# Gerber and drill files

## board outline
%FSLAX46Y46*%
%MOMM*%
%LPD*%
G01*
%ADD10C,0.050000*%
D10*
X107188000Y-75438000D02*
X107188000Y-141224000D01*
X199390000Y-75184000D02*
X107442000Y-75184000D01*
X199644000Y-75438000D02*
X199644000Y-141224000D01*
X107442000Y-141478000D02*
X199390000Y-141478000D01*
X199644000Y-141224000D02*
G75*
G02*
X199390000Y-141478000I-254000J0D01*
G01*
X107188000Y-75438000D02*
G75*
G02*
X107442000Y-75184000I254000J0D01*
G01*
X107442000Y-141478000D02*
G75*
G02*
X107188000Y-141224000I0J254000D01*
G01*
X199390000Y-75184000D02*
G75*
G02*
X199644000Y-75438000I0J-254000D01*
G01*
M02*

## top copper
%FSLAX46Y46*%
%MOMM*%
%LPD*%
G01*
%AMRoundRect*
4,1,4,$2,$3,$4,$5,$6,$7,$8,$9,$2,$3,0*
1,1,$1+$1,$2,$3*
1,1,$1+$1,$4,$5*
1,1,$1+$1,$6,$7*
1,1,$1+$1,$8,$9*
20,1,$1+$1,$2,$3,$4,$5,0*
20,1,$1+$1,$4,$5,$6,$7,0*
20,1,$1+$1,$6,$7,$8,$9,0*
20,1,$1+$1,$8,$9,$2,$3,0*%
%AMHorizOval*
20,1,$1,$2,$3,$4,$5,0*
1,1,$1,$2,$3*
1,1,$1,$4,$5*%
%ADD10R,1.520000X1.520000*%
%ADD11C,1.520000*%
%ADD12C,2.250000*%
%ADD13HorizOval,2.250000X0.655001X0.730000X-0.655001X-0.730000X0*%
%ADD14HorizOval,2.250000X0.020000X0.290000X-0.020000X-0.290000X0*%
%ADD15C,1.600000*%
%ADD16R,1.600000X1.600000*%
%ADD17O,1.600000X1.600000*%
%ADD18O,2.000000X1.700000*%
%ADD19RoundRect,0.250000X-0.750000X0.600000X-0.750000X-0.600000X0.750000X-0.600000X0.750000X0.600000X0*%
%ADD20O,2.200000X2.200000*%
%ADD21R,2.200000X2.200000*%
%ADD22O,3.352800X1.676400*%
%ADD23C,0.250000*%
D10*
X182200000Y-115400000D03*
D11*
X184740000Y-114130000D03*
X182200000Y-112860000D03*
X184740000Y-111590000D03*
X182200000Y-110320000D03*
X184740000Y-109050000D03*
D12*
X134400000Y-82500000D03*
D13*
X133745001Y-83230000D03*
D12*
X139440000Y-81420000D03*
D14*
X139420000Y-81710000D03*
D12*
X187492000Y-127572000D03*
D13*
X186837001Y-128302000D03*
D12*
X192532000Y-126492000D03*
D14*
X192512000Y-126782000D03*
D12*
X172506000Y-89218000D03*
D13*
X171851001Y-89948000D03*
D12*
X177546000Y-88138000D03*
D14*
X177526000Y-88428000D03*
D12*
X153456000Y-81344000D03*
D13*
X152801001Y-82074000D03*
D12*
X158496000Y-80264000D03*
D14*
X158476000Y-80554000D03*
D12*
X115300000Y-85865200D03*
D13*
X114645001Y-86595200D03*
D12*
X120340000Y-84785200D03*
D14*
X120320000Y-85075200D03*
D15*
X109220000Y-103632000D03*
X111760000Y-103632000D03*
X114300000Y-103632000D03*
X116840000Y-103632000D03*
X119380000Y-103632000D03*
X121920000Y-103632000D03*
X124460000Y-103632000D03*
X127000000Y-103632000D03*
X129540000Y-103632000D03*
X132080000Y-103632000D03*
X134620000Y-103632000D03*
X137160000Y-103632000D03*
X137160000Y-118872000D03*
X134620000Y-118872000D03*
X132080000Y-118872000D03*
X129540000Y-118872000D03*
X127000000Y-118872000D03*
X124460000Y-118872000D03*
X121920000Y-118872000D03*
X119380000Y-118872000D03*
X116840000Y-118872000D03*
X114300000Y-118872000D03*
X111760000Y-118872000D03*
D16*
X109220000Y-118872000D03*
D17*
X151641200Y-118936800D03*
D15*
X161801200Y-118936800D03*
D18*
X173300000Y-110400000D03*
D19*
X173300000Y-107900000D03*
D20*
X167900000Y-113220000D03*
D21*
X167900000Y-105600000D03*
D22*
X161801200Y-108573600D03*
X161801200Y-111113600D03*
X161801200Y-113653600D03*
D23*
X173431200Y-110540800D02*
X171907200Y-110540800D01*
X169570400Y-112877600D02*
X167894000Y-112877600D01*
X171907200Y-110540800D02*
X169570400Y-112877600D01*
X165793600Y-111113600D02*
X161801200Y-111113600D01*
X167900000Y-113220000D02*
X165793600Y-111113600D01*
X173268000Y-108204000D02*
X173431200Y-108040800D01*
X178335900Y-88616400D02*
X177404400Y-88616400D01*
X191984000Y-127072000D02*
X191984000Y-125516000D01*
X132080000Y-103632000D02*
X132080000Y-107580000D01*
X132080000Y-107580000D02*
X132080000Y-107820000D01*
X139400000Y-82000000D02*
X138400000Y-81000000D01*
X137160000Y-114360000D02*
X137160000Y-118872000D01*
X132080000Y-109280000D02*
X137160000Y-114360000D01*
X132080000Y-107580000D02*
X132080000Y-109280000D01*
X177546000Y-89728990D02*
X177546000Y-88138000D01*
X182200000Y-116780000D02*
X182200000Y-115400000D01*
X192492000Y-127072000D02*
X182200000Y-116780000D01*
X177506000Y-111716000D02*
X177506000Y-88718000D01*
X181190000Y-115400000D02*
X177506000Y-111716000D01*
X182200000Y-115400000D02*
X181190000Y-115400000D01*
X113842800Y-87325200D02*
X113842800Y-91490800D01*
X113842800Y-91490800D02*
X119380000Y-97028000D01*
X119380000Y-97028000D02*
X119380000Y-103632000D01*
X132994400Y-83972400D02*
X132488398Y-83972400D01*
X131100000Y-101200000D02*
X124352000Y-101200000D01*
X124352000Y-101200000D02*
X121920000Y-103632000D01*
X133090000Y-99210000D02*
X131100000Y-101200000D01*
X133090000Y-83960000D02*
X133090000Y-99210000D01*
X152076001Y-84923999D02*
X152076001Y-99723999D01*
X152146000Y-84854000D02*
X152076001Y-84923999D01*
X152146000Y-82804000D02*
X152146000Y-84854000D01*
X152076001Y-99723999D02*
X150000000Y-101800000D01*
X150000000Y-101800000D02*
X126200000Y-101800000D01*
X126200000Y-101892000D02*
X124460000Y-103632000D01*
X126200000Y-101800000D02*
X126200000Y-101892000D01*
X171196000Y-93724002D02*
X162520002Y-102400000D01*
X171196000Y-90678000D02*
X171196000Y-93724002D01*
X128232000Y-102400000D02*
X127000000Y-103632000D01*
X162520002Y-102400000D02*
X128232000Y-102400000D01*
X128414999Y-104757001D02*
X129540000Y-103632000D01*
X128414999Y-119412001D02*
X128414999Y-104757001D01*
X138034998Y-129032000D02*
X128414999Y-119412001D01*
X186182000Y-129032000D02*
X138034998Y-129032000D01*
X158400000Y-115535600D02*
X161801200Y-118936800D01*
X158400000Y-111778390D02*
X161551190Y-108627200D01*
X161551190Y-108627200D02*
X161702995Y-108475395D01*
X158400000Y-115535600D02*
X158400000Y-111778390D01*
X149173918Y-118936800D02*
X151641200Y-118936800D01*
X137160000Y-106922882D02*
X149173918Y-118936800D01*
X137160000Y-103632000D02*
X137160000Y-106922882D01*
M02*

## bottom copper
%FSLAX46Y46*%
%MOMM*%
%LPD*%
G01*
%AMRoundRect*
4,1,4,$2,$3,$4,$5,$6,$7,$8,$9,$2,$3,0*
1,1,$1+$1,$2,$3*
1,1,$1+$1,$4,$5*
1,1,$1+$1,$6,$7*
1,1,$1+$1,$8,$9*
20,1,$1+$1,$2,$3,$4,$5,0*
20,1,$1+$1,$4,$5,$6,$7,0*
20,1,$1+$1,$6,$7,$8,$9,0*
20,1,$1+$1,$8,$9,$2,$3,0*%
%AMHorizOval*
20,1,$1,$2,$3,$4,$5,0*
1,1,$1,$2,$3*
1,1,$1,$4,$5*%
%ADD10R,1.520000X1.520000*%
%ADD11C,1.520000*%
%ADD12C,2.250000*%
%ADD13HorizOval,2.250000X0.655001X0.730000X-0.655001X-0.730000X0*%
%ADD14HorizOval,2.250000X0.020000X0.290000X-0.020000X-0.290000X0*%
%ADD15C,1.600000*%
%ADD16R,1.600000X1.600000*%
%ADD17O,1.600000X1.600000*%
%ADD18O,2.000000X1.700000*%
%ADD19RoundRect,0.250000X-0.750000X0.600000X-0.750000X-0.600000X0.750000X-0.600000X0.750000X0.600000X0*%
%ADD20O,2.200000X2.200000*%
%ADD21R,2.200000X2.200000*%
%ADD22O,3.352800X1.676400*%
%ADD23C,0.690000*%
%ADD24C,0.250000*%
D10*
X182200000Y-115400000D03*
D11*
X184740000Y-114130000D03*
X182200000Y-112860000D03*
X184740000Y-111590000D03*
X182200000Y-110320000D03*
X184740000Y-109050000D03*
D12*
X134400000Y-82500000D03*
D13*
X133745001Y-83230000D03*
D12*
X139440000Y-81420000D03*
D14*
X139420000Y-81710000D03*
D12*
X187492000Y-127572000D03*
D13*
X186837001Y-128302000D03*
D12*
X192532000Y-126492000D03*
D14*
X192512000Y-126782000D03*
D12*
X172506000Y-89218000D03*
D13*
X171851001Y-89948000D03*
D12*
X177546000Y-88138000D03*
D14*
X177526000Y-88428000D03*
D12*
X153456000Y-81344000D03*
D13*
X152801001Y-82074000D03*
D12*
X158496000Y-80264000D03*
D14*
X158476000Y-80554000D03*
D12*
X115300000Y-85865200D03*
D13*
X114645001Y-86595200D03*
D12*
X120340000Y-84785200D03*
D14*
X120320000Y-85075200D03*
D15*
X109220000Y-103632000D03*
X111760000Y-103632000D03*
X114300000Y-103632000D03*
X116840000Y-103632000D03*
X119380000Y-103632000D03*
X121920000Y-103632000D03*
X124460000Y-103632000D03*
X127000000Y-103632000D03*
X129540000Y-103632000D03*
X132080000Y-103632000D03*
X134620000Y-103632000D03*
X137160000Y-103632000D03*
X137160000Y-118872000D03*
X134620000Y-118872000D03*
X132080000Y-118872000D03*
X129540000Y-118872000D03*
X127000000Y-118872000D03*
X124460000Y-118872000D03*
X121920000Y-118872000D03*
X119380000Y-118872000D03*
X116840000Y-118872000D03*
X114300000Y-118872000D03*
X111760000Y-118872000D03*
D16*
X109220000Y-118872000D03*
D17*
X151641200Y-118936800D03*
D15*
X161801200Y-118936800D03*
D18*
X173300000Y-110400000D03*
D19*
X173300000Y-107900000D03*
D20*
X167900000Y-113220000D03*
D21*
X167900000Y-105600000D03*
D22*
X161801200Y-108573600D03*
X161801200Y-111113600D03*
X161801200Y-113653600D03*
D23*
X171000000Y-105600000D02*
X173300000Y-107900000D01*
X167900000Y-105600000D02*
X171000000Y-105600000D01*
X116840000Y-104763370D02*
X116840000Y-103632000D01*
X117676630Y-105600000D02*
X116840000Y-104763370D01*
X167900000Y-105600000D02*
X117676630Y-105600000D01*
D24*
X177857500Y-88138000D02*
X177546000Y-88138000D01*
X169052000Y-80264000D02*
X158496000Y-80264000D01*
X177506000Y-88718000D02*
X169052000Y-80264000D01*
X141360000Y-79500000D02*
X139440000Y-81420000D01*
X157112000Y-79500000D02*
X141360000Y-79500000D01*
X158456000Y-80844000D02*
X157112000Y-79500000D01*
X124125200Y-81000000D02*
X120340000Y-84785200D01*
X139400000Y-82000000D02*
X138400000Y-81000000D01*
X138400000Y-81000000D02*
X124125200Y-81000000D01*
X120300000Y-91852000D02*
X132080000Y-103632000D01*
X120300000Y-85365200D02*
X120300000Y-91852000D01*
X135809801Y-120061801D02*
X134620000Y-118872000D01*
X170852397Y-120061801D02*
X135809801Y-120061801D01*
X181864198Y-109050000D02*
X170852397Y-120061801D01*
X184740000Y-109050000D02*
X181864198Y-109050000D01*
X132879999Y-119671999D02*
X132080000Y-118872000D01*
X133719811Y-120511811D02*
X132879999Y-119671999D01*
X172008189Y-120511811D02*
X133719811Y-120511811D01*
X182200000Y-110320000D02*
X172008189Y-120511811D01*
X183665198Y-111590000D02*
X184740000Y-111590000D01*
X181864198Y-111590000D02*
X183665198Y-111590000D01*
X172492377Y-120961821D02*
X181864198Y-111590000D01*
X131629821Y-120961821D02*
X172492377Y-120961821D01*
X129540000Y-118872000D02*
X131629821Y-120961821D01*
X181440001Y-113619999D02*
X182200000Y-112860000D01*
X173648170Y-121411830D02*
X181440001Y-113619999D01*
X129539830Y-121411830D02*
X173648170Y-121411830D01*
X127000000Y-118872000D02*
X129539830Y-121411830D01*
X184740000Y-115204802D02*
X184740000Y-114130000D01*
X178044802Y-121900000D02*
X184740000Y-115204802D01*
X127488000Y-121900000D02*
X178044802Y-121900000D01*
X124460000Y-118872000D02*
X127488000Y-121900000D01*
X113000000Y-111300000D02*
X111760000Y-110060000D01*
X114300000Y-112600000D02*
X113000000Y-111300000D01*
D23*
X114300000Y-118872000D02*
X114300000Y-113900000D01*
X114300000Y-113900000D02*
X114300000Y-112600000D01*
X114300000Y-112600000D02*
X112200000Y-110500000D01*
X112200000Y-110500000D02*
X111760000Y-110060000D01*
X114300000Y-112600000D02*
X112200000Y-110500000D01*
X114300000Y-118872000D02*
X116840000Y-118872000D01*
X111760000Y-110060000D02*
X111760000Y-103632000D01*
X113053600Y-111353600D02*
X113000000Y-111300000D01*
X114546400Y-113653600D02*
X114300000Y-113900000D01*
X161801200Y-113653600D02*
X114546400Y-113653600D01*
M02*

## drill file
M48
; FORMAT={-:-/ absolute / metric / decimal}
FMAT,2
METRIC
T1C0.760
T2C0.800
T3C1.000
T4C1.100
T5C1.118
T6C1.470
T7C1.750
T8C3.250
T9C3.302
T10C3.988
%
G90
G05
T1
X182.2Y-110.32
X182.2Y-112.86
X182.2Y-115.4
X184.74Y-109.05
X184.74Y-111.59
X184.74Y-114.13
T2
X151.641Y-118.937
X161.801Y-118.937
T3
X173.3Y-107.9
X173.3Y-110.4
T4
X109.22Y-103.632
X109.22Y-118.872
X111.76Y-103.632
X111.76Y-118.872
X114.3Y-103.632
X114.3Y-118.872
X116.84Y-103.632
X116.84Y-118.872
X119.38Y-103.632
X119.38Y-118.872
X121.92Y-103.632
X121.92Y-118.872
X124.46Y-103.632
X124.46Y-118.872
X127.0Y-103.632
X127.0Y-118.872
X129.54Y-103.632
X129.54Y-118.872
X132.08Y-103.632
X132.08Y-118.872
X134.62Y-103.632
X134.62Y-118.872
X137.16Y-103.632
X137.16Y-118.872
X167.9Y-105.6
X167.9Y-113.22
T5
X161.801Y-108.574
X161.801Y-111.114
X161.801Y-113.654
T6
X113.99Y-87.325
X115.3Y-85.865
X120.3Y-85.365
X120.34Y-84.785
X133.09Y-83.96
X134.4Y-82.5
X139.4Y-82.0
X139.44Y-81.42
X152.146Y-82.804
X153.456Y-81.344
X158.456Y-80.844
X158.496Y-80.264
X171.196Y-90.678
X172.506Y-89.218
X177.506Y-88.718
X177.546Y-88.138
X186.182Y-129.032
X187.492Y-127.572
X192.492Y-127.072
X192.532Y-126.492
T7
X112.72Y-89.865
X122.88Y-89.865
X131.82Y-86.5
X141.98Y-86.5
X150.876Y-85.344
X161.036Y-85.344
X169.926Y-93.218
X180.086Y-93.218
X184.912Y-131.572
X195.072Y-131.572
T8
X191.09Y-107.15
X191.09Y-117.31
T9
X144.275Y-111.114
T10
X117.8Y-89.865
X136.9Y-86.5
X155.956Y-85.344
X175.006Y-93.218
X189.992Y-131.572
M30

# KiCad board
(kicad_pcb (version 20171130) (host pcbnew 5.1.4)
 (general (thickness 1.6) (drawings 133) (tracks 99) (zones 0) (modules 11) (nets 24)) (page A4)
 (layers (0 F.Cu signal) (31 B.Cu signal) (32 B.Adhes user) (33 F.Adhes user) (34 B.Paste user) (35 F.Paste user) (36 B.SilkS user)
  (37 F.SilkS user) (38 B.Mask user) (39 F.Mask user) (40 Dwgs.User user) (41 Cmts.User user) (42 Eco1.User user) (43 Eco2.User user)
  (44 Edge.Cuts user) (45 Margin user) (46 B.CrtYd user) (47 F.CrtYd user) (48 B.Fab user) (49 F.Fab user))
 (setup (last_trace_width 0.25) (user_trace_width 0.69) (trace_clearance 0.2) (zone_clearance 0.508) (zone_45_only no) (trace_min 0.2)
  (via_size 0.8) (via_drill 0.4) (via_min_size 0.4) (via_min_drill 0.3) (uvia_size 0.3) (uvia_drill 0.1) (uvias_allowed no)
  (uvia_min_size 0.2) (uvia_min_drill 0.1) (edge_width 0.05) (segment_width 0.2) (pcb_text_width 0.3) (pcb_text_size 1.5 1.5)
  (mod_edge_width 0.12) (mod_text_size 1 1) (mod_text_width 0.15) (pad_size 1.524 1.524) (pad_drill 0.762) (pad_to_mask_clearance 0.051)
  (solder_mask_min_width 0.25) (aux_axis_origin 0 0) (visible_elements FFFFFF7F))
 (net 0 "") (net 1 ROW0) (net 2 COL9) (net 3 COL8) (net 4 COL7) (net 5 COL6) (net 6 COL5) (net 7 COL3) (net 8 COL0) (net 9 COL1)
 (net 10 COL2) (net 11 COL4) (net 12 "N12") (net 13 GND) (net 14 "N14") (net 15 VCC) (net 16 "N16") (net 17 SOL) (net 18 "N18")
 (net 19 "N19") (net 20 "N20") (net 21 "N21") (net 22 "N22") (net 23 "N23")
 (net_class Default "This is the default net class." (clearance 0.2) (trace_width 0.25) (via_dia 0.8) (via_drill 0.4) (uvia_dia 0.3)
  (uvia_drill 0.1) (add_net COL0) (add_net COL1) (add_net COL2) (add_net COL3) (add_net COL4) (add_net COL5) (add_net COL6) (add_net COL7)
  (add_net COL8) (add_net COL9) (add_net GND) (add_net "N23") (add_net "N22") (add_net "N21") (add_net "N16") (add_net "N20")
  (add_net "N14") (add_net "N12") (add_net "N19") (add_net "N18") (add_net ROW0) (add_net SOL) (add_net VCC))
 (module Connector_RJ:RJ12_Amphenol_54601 (layer F.Cu) (at 182.2 115.4 90)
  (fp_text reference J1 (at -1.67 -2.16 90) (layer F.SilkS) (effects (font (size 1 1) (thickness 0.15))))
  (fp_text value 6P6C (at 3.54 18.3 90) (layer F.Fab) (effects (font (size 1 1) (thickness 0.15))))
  (pad 1 thru_hole rect (at 0 0 90) (size 1.52 1.52) (drill 0.76) (layers *.Cu *.Mask) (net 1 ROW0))
  (pad "" np_thru_hole circle (at -1.91 8.89 90) (size 3.25 3.25) (drill 3.25) (layers *.Cu *.Mask))
  (pad 2 thru_hole circle (at 1.27 2.54 90) (size 1.52 1.52) (drill 0.76) (layers *.Cu *.Mask) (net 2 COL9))
  (pad 3 thru_hole circle (at 2.54 0 90) (size 1.52 1.52) (drill 0.76) (layers *.Cu *.Mask) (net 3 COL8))
  (pad 4 thru_hole circle (at 3.81 2.54 90) (size 1.52 1.52) (drill 0.76) (layers *.Cu *.Mask) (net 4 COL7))
  (pad 5 thru_hole circle (at 5.08 0 90) (size 1.52 1.52) (drill 0.76) (layers *.Cu *.Mask) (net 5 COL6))
  (pad 6 thru_hole circle (at 6.35 2.54 90) (size 1.52 1.52) (drill 0.76) (layers *.Cu *.Mask) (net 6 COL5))
  (pad "" np_thru_hole circle (at 8.25 8.89 90) (size 3.25 3.25) (drill 3.25) (layers *.Cu *.Mask)))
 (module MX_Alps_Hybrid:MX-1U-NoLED (layer F.Cu) (at 136.9 86.5)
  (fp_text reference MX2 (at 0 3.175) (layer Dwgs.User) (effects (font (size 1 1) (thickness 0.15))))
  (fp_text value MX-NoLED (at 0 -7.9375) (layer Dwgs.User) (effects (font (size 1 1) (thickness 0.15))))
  (pad "" np_thru_hole circle (at 5.08 0 48.0996) (size 1.75 1.75) (drill 1.75) (layers *.Cu *.Mask))
  (pad "" np_thru_hole circle (at -5.08 0 48.0996) (size 1.75 1.75) (drill 1.75) (layers *.Cu *.Mask))
  (pad 1 thru_hole circle (at -2.5 -4) (size 2.25 2.25) (drill 1.47) (layers *.Cu B.Mask) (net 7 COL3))
  (pad "" np_thru_hole circle (at 0 0) (size 3.9878 3.9878) (drill 3.9878) (layers *.Cu *.Mask))
  (pad 1 thru_hole oval (at -3.81 -2.54 48.0996) (size 4.211556 2.25) (drill 1.47 (offset 0.980778 0)) (layers *.Cu B.Mask) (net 7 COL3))
  (pad 2 thru_hole circle (at 2.54 -5.08) (size 2.25 2.25) (drill 1.47) (layers *.Cu B.Mask) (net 1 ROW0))
  (pad 2 thru_hole oval (at 2.5 -4.5 86.0548) (size 2.831378 2.25) (drill 1.47 (offset 0.290689 0)) (layers *.Cu B.Mask) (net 1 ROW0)))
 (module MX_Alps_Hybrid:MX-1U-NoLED (layer F.Cu) (at 189.992 131.572)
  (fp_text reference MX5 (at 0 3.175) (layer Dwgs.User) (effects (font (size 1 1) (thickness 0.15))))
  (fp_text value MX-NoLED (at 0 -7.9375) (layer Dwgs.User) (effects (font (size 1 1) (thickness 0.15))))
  (pad "" np_thru_hole circle (at 5.08 0 48.0996) (size 1.75 1.75) (drill 1.75) (layers *.Cu *.Mask))
  (pad "" np_thru_hole circle (at -5.08 0 48.0996) (size 1.75 1.75) (drill 1.75) (layers *.Cu *.Mask))
  (pad 1 thru_hole circle (at -2.5 -4) (size 2.25 2.25) (drill 1.47) (layers *.Cu B.Mask) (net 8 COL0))
  (pad "" np_thru_hole circle (at 0 0) (size 3.9878 3.9878) (drill 3.9878) (layers *.Cu *.Mask))
  (pad 1 thru_hole oval (at -3.81 -2.54 48.0996) (size 4.211556 2.25) (drill 1.47 (offset 0.980778 0)) (layers *.Cu B.Mask) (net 8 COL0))
  (pad 2 thru_hole circle (at 2.54 -5.08) (size 2.25 2.25) (drill 1.47) (layers *.Cu B.Mask) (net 1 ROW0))
  (pad 2 thru_hole oval (at 2.5 -4.5 86.0548) (size 2.831378 2.25) (drill 1.47 (offset 0.290689 0)) (layers *.Cu B.Mask) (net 1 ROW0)))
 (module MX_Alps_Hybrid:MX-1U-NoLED (layer F.Cu) (at 175.006 93.218)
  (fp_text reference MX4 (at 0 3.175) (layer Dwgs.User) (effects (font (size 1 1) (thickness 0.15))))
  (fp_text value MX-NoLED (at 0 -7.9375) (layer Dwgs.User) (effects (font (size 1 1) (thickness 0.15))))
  (pad "" np_thru_hole circle (at 5.08 0 48.0996) (size 1.75 1.75) (drill 1.75) (layers *.Cu *.Mask))
  (pad "" np_thru_hole circle (at -5.08 0 48.0996) (size 1.75 1.75) (drill 1.75) (layers *.Cu *.Mask))
  (pad 1 thru_hole circle (at -2.5 -4) (size 2.25 2.25) (drill 1.47) (layers *.Cu B.Mask) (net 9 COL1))
  (pad "" np_thru_hole circle (at 0 0) (size 3.9878 3.9878) (drill 3.9878) (layers *.Cu *.Mask))
  (pad 1 thru_hole oval (at -3.81 -2.54 48.0996) (size 4.211556 2.25) (drill 1.47 (offset 0.980778 0)) (layers *.Cu B.Mask) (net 9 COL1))
  (pad 2 thru_hole circle (at 2.54 -5.08) (size 2.25 2.25) (drill 1.47) (layers *.Cu B.Mask) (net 1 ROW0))
  (pad 2 thru_hole oval (at 2.5 -4.5 86.0548) (size 2.831378 2.25) (drill 1.47 (offset 0.290689 0)) (layers *.Cu B.Mask) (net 1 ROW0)))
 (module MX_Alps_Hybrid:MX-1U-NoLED (layer F.Cu) (at 155.956 85.344)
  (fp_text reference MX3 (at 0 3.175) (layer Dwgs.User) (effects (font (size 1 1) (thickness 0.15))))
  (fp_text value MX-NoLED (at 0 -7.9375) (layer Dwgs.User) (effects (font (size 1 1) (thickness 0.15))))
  (pad "" np_thru_hole circle (at 5.08 0 48.0996) (size 1.75 1.75) (drill 1.75) (layers *.Cu *.Mask))
  (pad "" np_thru_hole circle (at -5.08 0 48.0996) (size 1.75 1.75) (drill 1.75) (layers *.Cu *.Mask))
  (pad 1 thru_hole circle (at -2.5 -4) (size 2.25 2.25) (drill 1.47) (layers *.Cu B.Mask) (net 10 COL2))
  (pad "" np_thru_hole circle (at 0 0) (size 3.9878 3.9878) (drill 3.9878) (layers *.Cu *.Mask))
  (pad 1 thru_hole oval (at -3.81 -2.54 48.0996) (size 4.211556 2.25) (drill 1.47 (offset 0.980778 0)) (layers *.Cu B.Mask) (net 10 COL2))
  (pad 2 thru_hole circle (at 2.54 -5.08) (size 2.25 2.25) (drill 1.47) (layers *.Cu B.Mask) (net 1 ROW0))
  (pad 2 thru_hole oval (at 2.5 -4.5 86.0548) (size 2.831378 2.25) (drill 1.47 (offset 0.290689 0)) (layers *.Cu B.Mask) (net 1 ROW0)))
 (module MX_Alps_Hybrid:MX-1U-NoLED (layer F.Cu) (at 117.8 89.8652)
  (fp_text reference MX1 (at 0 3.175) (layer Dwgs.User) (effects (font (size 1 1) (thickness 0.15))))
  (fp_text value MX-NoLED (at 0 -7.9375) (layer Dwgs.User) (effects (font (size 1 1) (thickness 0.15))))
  (pad "" np_thru_hole circle (at 5.08 0 48.0996) (size 1.75 1.75) (drill 1.75) (layers *.Cu *.Mask))
  (pad "" np_thru_hole circle (at -5.08 0 48.0996) (size 1.75 1.75) (drill 1.75) (layers *.Cu *.Mask))
  (pad 1 thru_hole circle (at -2.5 -4) (size 2.25 2.25) (drill 1.47) (layers *.Cu B.Mask) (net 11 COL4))
  (pad "" np_thru_hole circle (at 0 0) (size 3.9878 3.9878) (drill 3.9878) (layers *.Cu *.Mask))
  (pad 1 thru_hole oval (at -3.81 -2.54 48.0996) (size 4.211556 2.25) (drill 1.47 (offset 0.980778 0)) (layers *.Cu B.Mask) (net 11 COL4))
  (pad 2 thru_hole circle (at 2.54 -5.08) (size 2.25 2.25) (drill 1.47) (layers *.Cu B.Mask) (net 1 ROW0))
  (pad 2 thru_hole oval (at 2.5 -4.5 86.0548) (size 2.831378 2.25) (drill 1.47 (offset 0.290689 0)) (layers *.Cu B.Mask) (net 1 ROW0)))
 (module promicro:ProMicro (layer F.Cu) (at 123.19 111.252)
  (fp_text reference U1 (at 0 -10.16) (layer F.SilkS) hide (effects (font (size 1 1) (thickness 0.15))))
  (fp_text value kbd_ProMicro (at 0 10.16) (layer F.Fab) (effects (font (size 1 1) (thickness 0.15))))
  (pad 24 thru_hole circle (at -13.97 -7.62) (size 1.6 1.6) (drill 1.1) (layers *.Cu *.Mask F.SilkS) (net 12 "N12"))
  (pad 23 thru_hole circle (at -11.43 -7.62) (size 1.6 1.6) (drill 1.1) (layers *.Cu *.Mask F.SilkS) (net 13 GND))
  (pad 22 thru_hole circle (at -8.89 -7.62) (size 1.6 1.6) (drill 1.1) (layers *.Cu *.Mask F.SilkS) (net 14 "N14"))
  (pad 21 thru_hole circle (at -6.35 -7.62) (size 1.6 1.6) (drill 1.1) (layers *.Cu *.Mask F.SilkS) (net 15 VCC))
  (pad 20 thru_hole circle (at -3.81 -7.62) (size 1.6 1.6) (drill 1.1) (layers *.Cu *.Mask F.SilkS) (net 11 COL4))
  (pad 19 thru_hole circle (at -1.27 -7.62) (size 1.6 1.6) (drill 1.1) (layers *.Cu *.Mask F.SilkS) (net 7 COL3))
  (pad 18 thru_hole circle (at 1.27 -7.62) (size 1.6 1.6) (drill 1.1) (layers *.Cu *.Mask F.SilkS) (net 10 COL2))
  (pad 17 thru_hole circle (at 3.81 -7.62) (size 1.6 1.6) (drill 1.1) (layers *.Cu *.Mask F.SilkS) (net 9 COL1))
  (pad 16 thru_hole circle (at 6.35 -7.62) (size 1.6 1.6) (drill 1.1) (layers *.Cu *.Mask F.SilkS) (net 8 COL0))
  (pad 15 thru_hole circle (at 8.89 -7.62) (size 1.6 1.6) (drill 1.1) (layers *.Cu *.Mask F.SilkS) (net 1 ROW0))
  (pad 14 thru_hole circle (at 11.43 -7.62) (size 1.6 1.6) (drill 1.1) (layers *.Cu *.Mask F.SilkS) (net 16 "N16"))
  (pad 13 thru_hole circle (at 13.97 -7.62) (size 1.6 1.6) (drill 1.1) (layers *.Cu *.Mask F.SilkS) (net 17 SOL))
  (pad 12 thru_hole circle (at 13.97 7.62) (size 1.6 1.6) (drill 1.1) (layers *.Cu *.Mask F.SilkS) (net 1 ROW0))
  (pad 11 thru_hole circle (at 11.43 7.62) (size 1.6 1.6) (drill 1.1) (layers *.Cu *.Mask F.SilkS) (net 6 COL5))
  (pad 10 thru_hole circle (at 8.89 7.62) (size 1.6 1.6) (drill 1.1) (layers *.Cu *.Mask F.SilkS) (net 5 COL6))
  (pad 9 thru_hole circle (at 6.35 7.62) (size 1.6 1.6) (drill 1.1) (layers *.Cu *.Mask F.SilkS) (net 4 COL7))
  (pad 8 thru_hole circle (at 3.81 7.62) (size 1.6 1.6) (drill 1.1) (layers *.Cu *.Mask F.SilkS) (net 3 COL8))
  (pad 7 thru_hole circle (at 1.27 7.62) (size 1.6 1.6) (drill 1.1) (layers *.Cu *.Mask F.SilkS) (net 2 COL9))
  (pad 6 thru_hole circle (at -1.27 7.62) (size 1.6 1.6) (drill 1.1) (layers *.Cu *.Mask F.SilkS) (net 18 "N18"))
  (pad 5 thru_hole circle (at -3.81 7.62) (size 1.6 1.6) (drill 1.1) (layers *.Cu *.Mask F.SilkS) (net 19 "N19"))
  (pad 4 thru_hole circle (at -6.35 7.62) (size 1.6 1.6) (drill 1.1) (layers *.Cu *.Mask F.SilkS) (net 13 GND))
  (pad 3 thru_hole circle (at -8.89 7.62) (size 1.6 1.6) (drill 1.1) (layers *.Cu *.Mask F.SilkS) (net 13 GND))
  (pad 2 thru_hole circle (at -11.43 7.62) (size 1.6 1.6) (drill 1.1) (layers *.Cu *.Mask F.SilkS) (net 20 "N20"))
  (pad 1 thru_hole rect (at -13.97 7.62) (size 1.6 1.6) (drill 1.1) (layers *.Cu *.Mask F.SilkS) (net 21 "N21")))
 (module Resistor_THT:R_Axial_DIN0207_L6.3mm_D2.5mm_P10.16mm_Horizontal (layer B.Cu) (at 161.8012 118.9368 180)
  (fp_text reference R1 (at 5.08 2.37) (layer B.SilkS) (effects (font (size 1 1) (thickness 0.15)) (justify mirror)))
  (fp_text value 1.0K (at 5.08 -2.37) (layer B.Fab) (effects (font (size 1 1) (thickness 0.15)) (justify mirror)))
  (pad 2 thru_hole oval (at 10.16 0 180) (size 1.6 1.6) (drill 0.8) (layers *.Cu *.Mask) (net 17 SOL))
  (pad 1 thru_hole circle (at 0 0 180) (size 1.6 1.6) (drill 0.8) (layers *.Cu *.Mask) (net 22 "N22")))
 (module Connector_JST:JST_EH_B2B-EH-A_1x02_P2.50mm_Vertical (layer B.Cu) (at 173.3 107.9 270)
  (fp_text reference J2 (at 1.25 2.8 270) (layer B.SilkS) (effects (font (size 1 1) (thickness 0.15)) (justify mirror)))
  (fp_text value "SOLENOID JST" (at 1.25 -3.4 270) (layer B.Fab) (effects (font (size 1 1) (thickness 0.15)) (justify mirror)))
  (pad 2 thru_hole oval (at 2.5 0 270) (size 1.7 2) (drill 1) (layers *.Cu *.Mask) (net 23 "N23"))
  (pad 1 thru_hole roundrect (at 0 0 270) (size 1.7 2) (drill 1) (layers *.Cu *.Mask) (roundrect_rratio 0.147059) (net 15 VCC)))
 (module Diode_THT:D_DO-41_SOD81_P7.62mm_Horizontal (layer B.Cu) (at 167.9 105.6 270)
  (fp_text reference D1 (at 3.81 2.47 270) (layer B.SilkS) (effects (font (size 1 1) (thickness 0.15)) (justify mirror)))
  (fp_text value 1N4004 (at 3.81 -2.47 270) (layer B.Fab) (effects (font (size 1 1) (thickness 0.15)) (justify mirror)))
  (pad 2 thru_hole oval (at 7.62 0 270) (size 2.2 2.2) (drill 1.1) (layers *.Cu *.Mask) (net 23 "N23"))
  (pad 1 thru_hole rect (at 0 0 270) (size 2.2 2.2) (drill 1.1) (layers *.Cu *.Mask) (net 15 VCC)))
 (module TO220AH (layer B.Cu) (at 155.4512 111.1136 270)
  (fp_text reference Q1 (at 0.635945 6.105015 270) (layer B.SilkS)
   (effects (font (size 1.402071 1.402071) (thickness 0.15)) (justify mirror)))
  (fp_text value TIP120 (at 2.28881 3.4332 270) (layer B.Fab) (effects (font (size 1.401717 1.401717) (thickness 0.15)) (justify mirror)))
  (pad B thru_hole oval (at -2.54 -6.35 270) (size 1.6764 3.3528) (drill 1.1176) (layers *.Cu *.Mask) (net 22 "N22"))
  (pad C thru_hole oval (at 0 -6.35 270) (size 1.6764 3.3528) (drill 1.1176) (layers *.Cu *.Mask) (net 23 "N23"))
  (pad E thru_hole oval (at 2.54 -6.35 270) (size 1.6764 3.3528) (drill 1.1176) (layers *.Cu *.Mask) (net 13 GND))
  (pad None np_thru_hole circle (at 0 11.176 270) (size 3.302 3.302) (drill 3.302) (layers *.Cu *.Mask)))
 (gr_line (start 107.188 75.438) (end 107.188 141.224) (layer Edge.Cuts) (width 0.05))
 (gr_line (start 199.39 75.184) (end 107.442 75.184) (layer Edge.Cuts) (width 0.05))
 (gr_line (start 199.644 75.438) (end 199.644 141.224) (layer Edge.Cuts) (width 0.05))
 (gr_line (start 107.442 141.478) (end 199.39 141.478) (layer Edge.Cuts) (width 0.05))
 (gr_arc (start 199.39 141.224) (end 199.39 141.478) (angle -90) (layer Edge.Cuts) (width 0.05))
 (gr_arc (start 107.442 75.438) (end 107.442 75.184) (angle -90) (layer Edge.Cuts) (width 0.05))
 (gr_arc (start 107.442 141.224) (end 107.188 141.224) (angle -90) (layer Edge.Cuts) (width 0.05))
 (gr_arc (start 199.39 75.438) (end 199.644 75.438) (angle -90) (layer Edge.Cuts) (width 0.05))
 (segment (start 173.4312 110.5408) (end 171.9072 110.5408) (width 0.25) (layer F.Cu) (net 23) (status 10))
 (segment (start 169.5704 112.8776) (end 167.894 112.8776) (width 0.25) (layer F.Cu) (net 23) (status 20))
 (segment (start 171.9072 110.5408) (end 169.5704 112.8776) (width 0.25) (layer F.Cu) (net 23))
 (segment (start 165.7936 111.1136) (end 161.8012 111.1136) (width 0.25) (layer F.Cu) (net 23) (status 20))
 (segment (start 167.9 113.22) (end 165.7936 111.1136) (width 0.25) (layer F.Cu) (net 23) (status 10))
 (segment (start 173.268 108.204) (end 173.4312 108.0408) (width 0.25) (layer F.Cu) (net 15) (status 30))
 (segment (start 171 105.6) (end 173.3 107.9) (width 0.69) (layer B.Cu) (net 15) (status 20))
 (segment (start 167.9 105.6) (end 171 105.6) (width 0.69) (layer B.Cu) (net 15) (status 10))
 (segment (start 116.84 104.76337) (end 116.84 103.632) (width 0.69) (layer B.Cu) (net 15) (status 20))
 (segment (start 117.67663 105.6) (end 116.84 104.76337) (width 0.69) (layer B.Cu) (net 15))
 (segment (start 167.9 105.6) (end 117.67663 105.6) (width 0.69) (layer B.Cu) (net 15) (status 10))
 (segment (start 178.3359 88.6164) (end 177.4044 88.6164) (width 0.25) (layer F.Cu) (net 1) (status 30))
 (segment (start 191.984 127.072) (end 191.984 125.516) (width 0.25) (layer F.Cu) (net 1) (status 30))
 (segment (start 132.08 103.632) (end 132.08 107.58) (width 0.25) (layer F.Cu) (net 1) (status 10))
 (segment (start 132.08 107.58) (end 132.08 107.82) (width 0.25) (layer F.Cu) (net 1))
 (segment (start 139.4 82) (end 138.4 81) (width 0.25) (layer F.Cu) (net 1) (status 30))
 (segment (start 177.8575 88.138) (end 177.546 88.138) (width 0.25) (layer B.Cu) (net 1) (status 30))
 (segment (start 169.052 80.264) (end 158.496 80.264) (width 0.25) (layer B.Cu) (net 1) (status 20))
 (segment (start 177.506 88.718) (end 169.052 80.264) (width 0.25) (layer B.Cu) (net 1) (status 10))
 (segment (start 141.36 79.5) (end 139.44 81.42) (width 0.25) (layer B.Cu) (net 1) (status 20))
 (segment (start 157.112 79.5) (end 141.36 79.5) (width 0.25) (layer B.Cu) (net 1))
 (segment (start 158.456 80.844) (end 157.112 79.5) (width 0.25) (layer B.Cu) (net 1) (status 10))
 (segment (start 124.1252 81) (end 120.34 84.7852) (width 0.25) (layer B.Cu) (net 1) (status 20))
 (segment (start 139.4 82) (end 138.4 81) (width 0.25) (layer B.Cu) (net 1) (status 30))
 (segment (start 138.4 81) (end 124.1252 81) (width 0.25) (layer B.Cu) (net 1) (status 10))
 (segment (start 120.3 91.852) (end 132.08 103.632) (width 0.25) (layer B.Cu) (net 1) (status 20))
 (segment (start 120.3 85.3652) (end 120.3 91.852) (width 0.25) (layer B.Cu) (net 1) (status 10))
 (segment (start 137.16 114.36) (end 137.16 118.872) (width 0.25) (layer F.Cu) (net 1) (status 20))
 (segment (start 132.08 109.28) (end 137.16 114.36) (width 0.25) (layer F.Cu) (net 1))
 (segment (start 132.08 107.58) (end 132.08 109.28) (width 0.25) (layer F.Cu) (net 1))
 (segment (start 177.546 89.72899) (end 177.546 88.138) (width 0.25) (layer F.Cu) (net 1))
 (segment (start 182.2 116.78) (end 182.2 115.4) (width 0.25) (layer F.Cu) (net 1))
 (segment (start 192.492 127.072) (end 182.2 116.78) (width 0.25) (layer F.Cu) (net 1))
 (segment (start 177.506 111.716) (end 177.506 88.718) (width 0.25) (layer F.Cu) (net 1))
 (segment (start 181.19 115.4) (end 177.506 111.716) (width 0.25) (layer F.Cu) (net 1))
 (segment (start 182.2 115.4) (end 181.19 115.4) (width 0.25) (layer F.Cu) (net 1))
 (segment (start 135.809801 120.061801) (end 134.62 118.872) (width 0.25) (layer B.Cu) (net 6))
 (segment (start 170.852397 120.061801) (end 135.809801 120.061801) (width 0.25) (layer B.Cu) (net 6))
 (segment (start 181.864198 109.05) (end 170.852397 120.061801) (width 0.25) (layer B.Cu) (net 6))
 (segment (start 184.74 109.05) (end 181.864198 109.05) (width 0.25) (layer B.Cu) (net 6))
 (segment (start 132.879999 119.671999) (end 132.08 118.872) (width 0.25) (layer B.Cu) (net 5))
 (segment (start 133.719811 120.511811) (end 132.879999 119.671999) (width 0.25) (layer B.Cu) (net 5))
 (segment (start 172.008189 120.511811) (end 133.719811 120.511811) (width 0.25) (layer B.Cu) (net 5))
 (segment (start 182.2 110.32) (end 172.008189 120.511811) (width 0.25) (layer B.Cu) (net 5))
 (segment (start 183.665198 111.59) (end 184.74 111.59) (width 0.25) (layer B.Cu) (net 4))
 (segment (start 181.864198 111.59) (end 183.665198 111.59) (width 0.25) (layer B.Cu) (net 4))
 (segment (start 172.492377 120.961821) (end 181.864198 111.59) (width 0.25) (layer B.Cu) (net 4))
 (segment (start 131.629821 120.961821) (end 172.492377 120.961821) (width 0.25) (layer B.Cu) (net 4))
 (segment (start 129.54 118.872) (end 131.629821 120.961821) (width 0.25) (layer B.Cu) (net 4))
 (segment (start 181.440001 113.619999) (end 182.2 112.86) (width 0.25) (layer B.Cu) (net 3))
 (segment (start 173.64817 121.41183) (end 181.440001 113.619999) (width 0.25) (layer B.Cu) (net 3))
 (segment (start 129.53983 121.41183) (end 173.64817 121.41183) (width 0.25) (layer B.Cu) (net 3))
 (segment (start 127 118.872) (end 129.53983 121.41183) (width 0.25) (layer B.Cu) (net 3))
 (segment (start 184.74 115.204802) (end 184.74 114.13) (width 0.25) (layer B.Cu) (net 2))
 (segment (start 178.044802 121.9) (end 184.74 115.204802) (width 0.25) (layer B.Cu) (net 2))
 (segment (start 127.488 121.9) (end 178.044802 121.9) (width 0.25) (layer B.Cu) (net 2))
 (segment (start 124.46 118.872) (end 127.488 121.9) (width 0.25) (layer B.Cu) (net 2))
 (segment (start 113.8428 87.3252) (end 113.8428 91.4908) (width 0.25) (layer F.Cu) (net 11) (status 10))
 (segment (start 113.8428 91.4908) (end 119.38 97.028) (width 0.25) (layer F.Cu) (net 11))
 (segment (start 119.38 97.028) (end 119.38 103.632) (width 0.25) (layer F.Cu) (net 11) (status 20))
 (segment (start 132.9944 83.9724) (end 132.488398 83.9724) (width 0.25) (layer F.Cu) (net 7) (status 30))
 (segment (start 131.1 101.2) (end 124.352 101.2) (width 0.25) (layer F.Cu) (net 7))
 (segment (start 124.352 101.2) (end 121.92 103.632) (width 0.25) (layer F.Cu) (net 7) (status 20))
 (segment (start 133.09 99.21) (end 131.1 101.2) (width 0.25) (layer F.Cu) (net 7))
 (segment (start 133.09 83.96) (end 133.09 99.21) (width 0.25) (layer F.Cu) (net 7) (status 10))
 (segment (start 152.076001 84.923999) (end 152.076001 99.723999) (width 0.25) (layer F.Cu) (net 10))
 (segment (start 152.146 84.854) (end 152.076001 84.923999) (width 0.25) (layer F.Cu) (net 10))
 (segment (start 152.146 82.804) (end 152.146 84.854) (width 0.25) (layer F.Cu) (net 10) (status 10))
 (segment (start 152.076001 99.723999) (end 150 101.8) (width 0.25) (layer F.Cu) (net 10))
 (segment (start 150 101.8) (end 126.2 101.8) (width 0.25) (layer F.Cu) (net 10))
 (segment (start 126.2 101.892) (end 124.46 103.632) (width 0.25) (layer F.Cu) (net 10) (status 20))
 (segment (start 126.2 101.8) (end 126.2 101.892) (width 0.25) (layer F.Cu) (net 10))
 (segment (start 171.196 93.724002) (end 162.520002 102.4) (width 0.25) (layer F.Cu) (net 9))
 (segment (start 171.196 90.678) (end 171.196 93.724002) (width 0.25) (layer F.Cu) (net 9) (status 10))
 (segment (start 128.232 102.4) (end 127 103.632) (width 0.25) (layer F.Cu) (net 9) (status 20))
 (segment (start 162.520002 102.4) (end 128.232 102.4) (width 0.25) (layer F.Cu) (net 9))
 (segment (start 128.414999 104.757001) (end 129.54 103.632) (width 0.25) (layer F.Cu) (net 8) (status 20))
 (segment (start 128.414999 119.412001) (end 128.414999 104.757001) (width 0.25) (layer F.Cu) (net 8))
 (segment (start 138.034998 129.032) (end 128.414999 119.412001) (width 0.25) (layer F.Cu) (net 8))
 (segment (start 186.182 129.032) (end 138.034998 129.032) (width 0.25) (layer F.Cu) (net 8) (status 10))
 (segment (start 113 111.3) (end 111.76 110.06) (width 0.25) (layer B.Cu) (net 13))
 (segment (start 114.3 112.6) (end 113 111.3) (width 0.25) (layer B.Cu) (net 13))
 (segment (start 114.3 118.872) (end 114.3 113.9) (width 0.69) (layer B.Cu) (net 13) (status 10))
 (segment (start 114.3 113.9) (end 114.3 112.6) (width 0.69) (layer B.Cu) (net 13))
 (segment (start 114.3 112.6) (end 112.2 110.5) (width 0.69) (layer B.Cu) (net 13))
 (segment (start 112.2 110.5) (end 111.76 110.06) (width 0.69) (layer B.Cu) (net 13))
 (segment (start 114.3 112.6) (end 112.2 110.5) (width 0.69) (layer B.Cu) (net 13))
 (segment (start 114.3 118.872) (end 116.84 118.872) (width 0.69) (layer B.Cu) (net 13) (status 30))
 (segment (start 111.76 110.06) (end 111.76 103.632) (width 0.69) (layer B.Cu) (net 13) (status 20))
 (segment (start 113.0536 111.3536) (end 113 111.3) (width 0.69) (layer B.Cu) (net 13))
 (segment (start 114.5464 113.6536) (end 114.3 113.9) (width 0.69) (layer B.Cu) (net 13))
 (segment (start 161.8012 113.6536) (end 114.5464 113.6536) (width 0.69) (layer B.Cu) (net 13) (status 10))
 (segment (start 158.4 115.5356) (end 161.8012 118.9368) (width 0.25) (layer F.Cu) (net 22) (status 20))
 (segment (start 158.4 111.77839) (end 161.55119 108.6272) (width 0.25) (layer F.Cu) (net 22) (status 20))
 (segment (start 161.55119 108.6272) (end 161.702995 108.475395) (width 0.25) (layer F.Cu) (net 22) (status 30))
 (segment (start 158.4 115.5356) (end 158.4 111.77839) (width 0.25) (layer F.Cu) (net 22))
 (segment (start 149.173918 118.9368) (end 151.6412 118.9368) (width 0.25) (layer F.Cu) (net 17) (status 20))
 (segment (start 137.16 106.922882) (end 149.173918 118.9368) (width 0.25) (layer F.Cu) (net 17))
 (segment (start 137.16 103.632) (end 137.16 106.922882) (width 0.25) (layer F.Cu) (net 17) (status 10)))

